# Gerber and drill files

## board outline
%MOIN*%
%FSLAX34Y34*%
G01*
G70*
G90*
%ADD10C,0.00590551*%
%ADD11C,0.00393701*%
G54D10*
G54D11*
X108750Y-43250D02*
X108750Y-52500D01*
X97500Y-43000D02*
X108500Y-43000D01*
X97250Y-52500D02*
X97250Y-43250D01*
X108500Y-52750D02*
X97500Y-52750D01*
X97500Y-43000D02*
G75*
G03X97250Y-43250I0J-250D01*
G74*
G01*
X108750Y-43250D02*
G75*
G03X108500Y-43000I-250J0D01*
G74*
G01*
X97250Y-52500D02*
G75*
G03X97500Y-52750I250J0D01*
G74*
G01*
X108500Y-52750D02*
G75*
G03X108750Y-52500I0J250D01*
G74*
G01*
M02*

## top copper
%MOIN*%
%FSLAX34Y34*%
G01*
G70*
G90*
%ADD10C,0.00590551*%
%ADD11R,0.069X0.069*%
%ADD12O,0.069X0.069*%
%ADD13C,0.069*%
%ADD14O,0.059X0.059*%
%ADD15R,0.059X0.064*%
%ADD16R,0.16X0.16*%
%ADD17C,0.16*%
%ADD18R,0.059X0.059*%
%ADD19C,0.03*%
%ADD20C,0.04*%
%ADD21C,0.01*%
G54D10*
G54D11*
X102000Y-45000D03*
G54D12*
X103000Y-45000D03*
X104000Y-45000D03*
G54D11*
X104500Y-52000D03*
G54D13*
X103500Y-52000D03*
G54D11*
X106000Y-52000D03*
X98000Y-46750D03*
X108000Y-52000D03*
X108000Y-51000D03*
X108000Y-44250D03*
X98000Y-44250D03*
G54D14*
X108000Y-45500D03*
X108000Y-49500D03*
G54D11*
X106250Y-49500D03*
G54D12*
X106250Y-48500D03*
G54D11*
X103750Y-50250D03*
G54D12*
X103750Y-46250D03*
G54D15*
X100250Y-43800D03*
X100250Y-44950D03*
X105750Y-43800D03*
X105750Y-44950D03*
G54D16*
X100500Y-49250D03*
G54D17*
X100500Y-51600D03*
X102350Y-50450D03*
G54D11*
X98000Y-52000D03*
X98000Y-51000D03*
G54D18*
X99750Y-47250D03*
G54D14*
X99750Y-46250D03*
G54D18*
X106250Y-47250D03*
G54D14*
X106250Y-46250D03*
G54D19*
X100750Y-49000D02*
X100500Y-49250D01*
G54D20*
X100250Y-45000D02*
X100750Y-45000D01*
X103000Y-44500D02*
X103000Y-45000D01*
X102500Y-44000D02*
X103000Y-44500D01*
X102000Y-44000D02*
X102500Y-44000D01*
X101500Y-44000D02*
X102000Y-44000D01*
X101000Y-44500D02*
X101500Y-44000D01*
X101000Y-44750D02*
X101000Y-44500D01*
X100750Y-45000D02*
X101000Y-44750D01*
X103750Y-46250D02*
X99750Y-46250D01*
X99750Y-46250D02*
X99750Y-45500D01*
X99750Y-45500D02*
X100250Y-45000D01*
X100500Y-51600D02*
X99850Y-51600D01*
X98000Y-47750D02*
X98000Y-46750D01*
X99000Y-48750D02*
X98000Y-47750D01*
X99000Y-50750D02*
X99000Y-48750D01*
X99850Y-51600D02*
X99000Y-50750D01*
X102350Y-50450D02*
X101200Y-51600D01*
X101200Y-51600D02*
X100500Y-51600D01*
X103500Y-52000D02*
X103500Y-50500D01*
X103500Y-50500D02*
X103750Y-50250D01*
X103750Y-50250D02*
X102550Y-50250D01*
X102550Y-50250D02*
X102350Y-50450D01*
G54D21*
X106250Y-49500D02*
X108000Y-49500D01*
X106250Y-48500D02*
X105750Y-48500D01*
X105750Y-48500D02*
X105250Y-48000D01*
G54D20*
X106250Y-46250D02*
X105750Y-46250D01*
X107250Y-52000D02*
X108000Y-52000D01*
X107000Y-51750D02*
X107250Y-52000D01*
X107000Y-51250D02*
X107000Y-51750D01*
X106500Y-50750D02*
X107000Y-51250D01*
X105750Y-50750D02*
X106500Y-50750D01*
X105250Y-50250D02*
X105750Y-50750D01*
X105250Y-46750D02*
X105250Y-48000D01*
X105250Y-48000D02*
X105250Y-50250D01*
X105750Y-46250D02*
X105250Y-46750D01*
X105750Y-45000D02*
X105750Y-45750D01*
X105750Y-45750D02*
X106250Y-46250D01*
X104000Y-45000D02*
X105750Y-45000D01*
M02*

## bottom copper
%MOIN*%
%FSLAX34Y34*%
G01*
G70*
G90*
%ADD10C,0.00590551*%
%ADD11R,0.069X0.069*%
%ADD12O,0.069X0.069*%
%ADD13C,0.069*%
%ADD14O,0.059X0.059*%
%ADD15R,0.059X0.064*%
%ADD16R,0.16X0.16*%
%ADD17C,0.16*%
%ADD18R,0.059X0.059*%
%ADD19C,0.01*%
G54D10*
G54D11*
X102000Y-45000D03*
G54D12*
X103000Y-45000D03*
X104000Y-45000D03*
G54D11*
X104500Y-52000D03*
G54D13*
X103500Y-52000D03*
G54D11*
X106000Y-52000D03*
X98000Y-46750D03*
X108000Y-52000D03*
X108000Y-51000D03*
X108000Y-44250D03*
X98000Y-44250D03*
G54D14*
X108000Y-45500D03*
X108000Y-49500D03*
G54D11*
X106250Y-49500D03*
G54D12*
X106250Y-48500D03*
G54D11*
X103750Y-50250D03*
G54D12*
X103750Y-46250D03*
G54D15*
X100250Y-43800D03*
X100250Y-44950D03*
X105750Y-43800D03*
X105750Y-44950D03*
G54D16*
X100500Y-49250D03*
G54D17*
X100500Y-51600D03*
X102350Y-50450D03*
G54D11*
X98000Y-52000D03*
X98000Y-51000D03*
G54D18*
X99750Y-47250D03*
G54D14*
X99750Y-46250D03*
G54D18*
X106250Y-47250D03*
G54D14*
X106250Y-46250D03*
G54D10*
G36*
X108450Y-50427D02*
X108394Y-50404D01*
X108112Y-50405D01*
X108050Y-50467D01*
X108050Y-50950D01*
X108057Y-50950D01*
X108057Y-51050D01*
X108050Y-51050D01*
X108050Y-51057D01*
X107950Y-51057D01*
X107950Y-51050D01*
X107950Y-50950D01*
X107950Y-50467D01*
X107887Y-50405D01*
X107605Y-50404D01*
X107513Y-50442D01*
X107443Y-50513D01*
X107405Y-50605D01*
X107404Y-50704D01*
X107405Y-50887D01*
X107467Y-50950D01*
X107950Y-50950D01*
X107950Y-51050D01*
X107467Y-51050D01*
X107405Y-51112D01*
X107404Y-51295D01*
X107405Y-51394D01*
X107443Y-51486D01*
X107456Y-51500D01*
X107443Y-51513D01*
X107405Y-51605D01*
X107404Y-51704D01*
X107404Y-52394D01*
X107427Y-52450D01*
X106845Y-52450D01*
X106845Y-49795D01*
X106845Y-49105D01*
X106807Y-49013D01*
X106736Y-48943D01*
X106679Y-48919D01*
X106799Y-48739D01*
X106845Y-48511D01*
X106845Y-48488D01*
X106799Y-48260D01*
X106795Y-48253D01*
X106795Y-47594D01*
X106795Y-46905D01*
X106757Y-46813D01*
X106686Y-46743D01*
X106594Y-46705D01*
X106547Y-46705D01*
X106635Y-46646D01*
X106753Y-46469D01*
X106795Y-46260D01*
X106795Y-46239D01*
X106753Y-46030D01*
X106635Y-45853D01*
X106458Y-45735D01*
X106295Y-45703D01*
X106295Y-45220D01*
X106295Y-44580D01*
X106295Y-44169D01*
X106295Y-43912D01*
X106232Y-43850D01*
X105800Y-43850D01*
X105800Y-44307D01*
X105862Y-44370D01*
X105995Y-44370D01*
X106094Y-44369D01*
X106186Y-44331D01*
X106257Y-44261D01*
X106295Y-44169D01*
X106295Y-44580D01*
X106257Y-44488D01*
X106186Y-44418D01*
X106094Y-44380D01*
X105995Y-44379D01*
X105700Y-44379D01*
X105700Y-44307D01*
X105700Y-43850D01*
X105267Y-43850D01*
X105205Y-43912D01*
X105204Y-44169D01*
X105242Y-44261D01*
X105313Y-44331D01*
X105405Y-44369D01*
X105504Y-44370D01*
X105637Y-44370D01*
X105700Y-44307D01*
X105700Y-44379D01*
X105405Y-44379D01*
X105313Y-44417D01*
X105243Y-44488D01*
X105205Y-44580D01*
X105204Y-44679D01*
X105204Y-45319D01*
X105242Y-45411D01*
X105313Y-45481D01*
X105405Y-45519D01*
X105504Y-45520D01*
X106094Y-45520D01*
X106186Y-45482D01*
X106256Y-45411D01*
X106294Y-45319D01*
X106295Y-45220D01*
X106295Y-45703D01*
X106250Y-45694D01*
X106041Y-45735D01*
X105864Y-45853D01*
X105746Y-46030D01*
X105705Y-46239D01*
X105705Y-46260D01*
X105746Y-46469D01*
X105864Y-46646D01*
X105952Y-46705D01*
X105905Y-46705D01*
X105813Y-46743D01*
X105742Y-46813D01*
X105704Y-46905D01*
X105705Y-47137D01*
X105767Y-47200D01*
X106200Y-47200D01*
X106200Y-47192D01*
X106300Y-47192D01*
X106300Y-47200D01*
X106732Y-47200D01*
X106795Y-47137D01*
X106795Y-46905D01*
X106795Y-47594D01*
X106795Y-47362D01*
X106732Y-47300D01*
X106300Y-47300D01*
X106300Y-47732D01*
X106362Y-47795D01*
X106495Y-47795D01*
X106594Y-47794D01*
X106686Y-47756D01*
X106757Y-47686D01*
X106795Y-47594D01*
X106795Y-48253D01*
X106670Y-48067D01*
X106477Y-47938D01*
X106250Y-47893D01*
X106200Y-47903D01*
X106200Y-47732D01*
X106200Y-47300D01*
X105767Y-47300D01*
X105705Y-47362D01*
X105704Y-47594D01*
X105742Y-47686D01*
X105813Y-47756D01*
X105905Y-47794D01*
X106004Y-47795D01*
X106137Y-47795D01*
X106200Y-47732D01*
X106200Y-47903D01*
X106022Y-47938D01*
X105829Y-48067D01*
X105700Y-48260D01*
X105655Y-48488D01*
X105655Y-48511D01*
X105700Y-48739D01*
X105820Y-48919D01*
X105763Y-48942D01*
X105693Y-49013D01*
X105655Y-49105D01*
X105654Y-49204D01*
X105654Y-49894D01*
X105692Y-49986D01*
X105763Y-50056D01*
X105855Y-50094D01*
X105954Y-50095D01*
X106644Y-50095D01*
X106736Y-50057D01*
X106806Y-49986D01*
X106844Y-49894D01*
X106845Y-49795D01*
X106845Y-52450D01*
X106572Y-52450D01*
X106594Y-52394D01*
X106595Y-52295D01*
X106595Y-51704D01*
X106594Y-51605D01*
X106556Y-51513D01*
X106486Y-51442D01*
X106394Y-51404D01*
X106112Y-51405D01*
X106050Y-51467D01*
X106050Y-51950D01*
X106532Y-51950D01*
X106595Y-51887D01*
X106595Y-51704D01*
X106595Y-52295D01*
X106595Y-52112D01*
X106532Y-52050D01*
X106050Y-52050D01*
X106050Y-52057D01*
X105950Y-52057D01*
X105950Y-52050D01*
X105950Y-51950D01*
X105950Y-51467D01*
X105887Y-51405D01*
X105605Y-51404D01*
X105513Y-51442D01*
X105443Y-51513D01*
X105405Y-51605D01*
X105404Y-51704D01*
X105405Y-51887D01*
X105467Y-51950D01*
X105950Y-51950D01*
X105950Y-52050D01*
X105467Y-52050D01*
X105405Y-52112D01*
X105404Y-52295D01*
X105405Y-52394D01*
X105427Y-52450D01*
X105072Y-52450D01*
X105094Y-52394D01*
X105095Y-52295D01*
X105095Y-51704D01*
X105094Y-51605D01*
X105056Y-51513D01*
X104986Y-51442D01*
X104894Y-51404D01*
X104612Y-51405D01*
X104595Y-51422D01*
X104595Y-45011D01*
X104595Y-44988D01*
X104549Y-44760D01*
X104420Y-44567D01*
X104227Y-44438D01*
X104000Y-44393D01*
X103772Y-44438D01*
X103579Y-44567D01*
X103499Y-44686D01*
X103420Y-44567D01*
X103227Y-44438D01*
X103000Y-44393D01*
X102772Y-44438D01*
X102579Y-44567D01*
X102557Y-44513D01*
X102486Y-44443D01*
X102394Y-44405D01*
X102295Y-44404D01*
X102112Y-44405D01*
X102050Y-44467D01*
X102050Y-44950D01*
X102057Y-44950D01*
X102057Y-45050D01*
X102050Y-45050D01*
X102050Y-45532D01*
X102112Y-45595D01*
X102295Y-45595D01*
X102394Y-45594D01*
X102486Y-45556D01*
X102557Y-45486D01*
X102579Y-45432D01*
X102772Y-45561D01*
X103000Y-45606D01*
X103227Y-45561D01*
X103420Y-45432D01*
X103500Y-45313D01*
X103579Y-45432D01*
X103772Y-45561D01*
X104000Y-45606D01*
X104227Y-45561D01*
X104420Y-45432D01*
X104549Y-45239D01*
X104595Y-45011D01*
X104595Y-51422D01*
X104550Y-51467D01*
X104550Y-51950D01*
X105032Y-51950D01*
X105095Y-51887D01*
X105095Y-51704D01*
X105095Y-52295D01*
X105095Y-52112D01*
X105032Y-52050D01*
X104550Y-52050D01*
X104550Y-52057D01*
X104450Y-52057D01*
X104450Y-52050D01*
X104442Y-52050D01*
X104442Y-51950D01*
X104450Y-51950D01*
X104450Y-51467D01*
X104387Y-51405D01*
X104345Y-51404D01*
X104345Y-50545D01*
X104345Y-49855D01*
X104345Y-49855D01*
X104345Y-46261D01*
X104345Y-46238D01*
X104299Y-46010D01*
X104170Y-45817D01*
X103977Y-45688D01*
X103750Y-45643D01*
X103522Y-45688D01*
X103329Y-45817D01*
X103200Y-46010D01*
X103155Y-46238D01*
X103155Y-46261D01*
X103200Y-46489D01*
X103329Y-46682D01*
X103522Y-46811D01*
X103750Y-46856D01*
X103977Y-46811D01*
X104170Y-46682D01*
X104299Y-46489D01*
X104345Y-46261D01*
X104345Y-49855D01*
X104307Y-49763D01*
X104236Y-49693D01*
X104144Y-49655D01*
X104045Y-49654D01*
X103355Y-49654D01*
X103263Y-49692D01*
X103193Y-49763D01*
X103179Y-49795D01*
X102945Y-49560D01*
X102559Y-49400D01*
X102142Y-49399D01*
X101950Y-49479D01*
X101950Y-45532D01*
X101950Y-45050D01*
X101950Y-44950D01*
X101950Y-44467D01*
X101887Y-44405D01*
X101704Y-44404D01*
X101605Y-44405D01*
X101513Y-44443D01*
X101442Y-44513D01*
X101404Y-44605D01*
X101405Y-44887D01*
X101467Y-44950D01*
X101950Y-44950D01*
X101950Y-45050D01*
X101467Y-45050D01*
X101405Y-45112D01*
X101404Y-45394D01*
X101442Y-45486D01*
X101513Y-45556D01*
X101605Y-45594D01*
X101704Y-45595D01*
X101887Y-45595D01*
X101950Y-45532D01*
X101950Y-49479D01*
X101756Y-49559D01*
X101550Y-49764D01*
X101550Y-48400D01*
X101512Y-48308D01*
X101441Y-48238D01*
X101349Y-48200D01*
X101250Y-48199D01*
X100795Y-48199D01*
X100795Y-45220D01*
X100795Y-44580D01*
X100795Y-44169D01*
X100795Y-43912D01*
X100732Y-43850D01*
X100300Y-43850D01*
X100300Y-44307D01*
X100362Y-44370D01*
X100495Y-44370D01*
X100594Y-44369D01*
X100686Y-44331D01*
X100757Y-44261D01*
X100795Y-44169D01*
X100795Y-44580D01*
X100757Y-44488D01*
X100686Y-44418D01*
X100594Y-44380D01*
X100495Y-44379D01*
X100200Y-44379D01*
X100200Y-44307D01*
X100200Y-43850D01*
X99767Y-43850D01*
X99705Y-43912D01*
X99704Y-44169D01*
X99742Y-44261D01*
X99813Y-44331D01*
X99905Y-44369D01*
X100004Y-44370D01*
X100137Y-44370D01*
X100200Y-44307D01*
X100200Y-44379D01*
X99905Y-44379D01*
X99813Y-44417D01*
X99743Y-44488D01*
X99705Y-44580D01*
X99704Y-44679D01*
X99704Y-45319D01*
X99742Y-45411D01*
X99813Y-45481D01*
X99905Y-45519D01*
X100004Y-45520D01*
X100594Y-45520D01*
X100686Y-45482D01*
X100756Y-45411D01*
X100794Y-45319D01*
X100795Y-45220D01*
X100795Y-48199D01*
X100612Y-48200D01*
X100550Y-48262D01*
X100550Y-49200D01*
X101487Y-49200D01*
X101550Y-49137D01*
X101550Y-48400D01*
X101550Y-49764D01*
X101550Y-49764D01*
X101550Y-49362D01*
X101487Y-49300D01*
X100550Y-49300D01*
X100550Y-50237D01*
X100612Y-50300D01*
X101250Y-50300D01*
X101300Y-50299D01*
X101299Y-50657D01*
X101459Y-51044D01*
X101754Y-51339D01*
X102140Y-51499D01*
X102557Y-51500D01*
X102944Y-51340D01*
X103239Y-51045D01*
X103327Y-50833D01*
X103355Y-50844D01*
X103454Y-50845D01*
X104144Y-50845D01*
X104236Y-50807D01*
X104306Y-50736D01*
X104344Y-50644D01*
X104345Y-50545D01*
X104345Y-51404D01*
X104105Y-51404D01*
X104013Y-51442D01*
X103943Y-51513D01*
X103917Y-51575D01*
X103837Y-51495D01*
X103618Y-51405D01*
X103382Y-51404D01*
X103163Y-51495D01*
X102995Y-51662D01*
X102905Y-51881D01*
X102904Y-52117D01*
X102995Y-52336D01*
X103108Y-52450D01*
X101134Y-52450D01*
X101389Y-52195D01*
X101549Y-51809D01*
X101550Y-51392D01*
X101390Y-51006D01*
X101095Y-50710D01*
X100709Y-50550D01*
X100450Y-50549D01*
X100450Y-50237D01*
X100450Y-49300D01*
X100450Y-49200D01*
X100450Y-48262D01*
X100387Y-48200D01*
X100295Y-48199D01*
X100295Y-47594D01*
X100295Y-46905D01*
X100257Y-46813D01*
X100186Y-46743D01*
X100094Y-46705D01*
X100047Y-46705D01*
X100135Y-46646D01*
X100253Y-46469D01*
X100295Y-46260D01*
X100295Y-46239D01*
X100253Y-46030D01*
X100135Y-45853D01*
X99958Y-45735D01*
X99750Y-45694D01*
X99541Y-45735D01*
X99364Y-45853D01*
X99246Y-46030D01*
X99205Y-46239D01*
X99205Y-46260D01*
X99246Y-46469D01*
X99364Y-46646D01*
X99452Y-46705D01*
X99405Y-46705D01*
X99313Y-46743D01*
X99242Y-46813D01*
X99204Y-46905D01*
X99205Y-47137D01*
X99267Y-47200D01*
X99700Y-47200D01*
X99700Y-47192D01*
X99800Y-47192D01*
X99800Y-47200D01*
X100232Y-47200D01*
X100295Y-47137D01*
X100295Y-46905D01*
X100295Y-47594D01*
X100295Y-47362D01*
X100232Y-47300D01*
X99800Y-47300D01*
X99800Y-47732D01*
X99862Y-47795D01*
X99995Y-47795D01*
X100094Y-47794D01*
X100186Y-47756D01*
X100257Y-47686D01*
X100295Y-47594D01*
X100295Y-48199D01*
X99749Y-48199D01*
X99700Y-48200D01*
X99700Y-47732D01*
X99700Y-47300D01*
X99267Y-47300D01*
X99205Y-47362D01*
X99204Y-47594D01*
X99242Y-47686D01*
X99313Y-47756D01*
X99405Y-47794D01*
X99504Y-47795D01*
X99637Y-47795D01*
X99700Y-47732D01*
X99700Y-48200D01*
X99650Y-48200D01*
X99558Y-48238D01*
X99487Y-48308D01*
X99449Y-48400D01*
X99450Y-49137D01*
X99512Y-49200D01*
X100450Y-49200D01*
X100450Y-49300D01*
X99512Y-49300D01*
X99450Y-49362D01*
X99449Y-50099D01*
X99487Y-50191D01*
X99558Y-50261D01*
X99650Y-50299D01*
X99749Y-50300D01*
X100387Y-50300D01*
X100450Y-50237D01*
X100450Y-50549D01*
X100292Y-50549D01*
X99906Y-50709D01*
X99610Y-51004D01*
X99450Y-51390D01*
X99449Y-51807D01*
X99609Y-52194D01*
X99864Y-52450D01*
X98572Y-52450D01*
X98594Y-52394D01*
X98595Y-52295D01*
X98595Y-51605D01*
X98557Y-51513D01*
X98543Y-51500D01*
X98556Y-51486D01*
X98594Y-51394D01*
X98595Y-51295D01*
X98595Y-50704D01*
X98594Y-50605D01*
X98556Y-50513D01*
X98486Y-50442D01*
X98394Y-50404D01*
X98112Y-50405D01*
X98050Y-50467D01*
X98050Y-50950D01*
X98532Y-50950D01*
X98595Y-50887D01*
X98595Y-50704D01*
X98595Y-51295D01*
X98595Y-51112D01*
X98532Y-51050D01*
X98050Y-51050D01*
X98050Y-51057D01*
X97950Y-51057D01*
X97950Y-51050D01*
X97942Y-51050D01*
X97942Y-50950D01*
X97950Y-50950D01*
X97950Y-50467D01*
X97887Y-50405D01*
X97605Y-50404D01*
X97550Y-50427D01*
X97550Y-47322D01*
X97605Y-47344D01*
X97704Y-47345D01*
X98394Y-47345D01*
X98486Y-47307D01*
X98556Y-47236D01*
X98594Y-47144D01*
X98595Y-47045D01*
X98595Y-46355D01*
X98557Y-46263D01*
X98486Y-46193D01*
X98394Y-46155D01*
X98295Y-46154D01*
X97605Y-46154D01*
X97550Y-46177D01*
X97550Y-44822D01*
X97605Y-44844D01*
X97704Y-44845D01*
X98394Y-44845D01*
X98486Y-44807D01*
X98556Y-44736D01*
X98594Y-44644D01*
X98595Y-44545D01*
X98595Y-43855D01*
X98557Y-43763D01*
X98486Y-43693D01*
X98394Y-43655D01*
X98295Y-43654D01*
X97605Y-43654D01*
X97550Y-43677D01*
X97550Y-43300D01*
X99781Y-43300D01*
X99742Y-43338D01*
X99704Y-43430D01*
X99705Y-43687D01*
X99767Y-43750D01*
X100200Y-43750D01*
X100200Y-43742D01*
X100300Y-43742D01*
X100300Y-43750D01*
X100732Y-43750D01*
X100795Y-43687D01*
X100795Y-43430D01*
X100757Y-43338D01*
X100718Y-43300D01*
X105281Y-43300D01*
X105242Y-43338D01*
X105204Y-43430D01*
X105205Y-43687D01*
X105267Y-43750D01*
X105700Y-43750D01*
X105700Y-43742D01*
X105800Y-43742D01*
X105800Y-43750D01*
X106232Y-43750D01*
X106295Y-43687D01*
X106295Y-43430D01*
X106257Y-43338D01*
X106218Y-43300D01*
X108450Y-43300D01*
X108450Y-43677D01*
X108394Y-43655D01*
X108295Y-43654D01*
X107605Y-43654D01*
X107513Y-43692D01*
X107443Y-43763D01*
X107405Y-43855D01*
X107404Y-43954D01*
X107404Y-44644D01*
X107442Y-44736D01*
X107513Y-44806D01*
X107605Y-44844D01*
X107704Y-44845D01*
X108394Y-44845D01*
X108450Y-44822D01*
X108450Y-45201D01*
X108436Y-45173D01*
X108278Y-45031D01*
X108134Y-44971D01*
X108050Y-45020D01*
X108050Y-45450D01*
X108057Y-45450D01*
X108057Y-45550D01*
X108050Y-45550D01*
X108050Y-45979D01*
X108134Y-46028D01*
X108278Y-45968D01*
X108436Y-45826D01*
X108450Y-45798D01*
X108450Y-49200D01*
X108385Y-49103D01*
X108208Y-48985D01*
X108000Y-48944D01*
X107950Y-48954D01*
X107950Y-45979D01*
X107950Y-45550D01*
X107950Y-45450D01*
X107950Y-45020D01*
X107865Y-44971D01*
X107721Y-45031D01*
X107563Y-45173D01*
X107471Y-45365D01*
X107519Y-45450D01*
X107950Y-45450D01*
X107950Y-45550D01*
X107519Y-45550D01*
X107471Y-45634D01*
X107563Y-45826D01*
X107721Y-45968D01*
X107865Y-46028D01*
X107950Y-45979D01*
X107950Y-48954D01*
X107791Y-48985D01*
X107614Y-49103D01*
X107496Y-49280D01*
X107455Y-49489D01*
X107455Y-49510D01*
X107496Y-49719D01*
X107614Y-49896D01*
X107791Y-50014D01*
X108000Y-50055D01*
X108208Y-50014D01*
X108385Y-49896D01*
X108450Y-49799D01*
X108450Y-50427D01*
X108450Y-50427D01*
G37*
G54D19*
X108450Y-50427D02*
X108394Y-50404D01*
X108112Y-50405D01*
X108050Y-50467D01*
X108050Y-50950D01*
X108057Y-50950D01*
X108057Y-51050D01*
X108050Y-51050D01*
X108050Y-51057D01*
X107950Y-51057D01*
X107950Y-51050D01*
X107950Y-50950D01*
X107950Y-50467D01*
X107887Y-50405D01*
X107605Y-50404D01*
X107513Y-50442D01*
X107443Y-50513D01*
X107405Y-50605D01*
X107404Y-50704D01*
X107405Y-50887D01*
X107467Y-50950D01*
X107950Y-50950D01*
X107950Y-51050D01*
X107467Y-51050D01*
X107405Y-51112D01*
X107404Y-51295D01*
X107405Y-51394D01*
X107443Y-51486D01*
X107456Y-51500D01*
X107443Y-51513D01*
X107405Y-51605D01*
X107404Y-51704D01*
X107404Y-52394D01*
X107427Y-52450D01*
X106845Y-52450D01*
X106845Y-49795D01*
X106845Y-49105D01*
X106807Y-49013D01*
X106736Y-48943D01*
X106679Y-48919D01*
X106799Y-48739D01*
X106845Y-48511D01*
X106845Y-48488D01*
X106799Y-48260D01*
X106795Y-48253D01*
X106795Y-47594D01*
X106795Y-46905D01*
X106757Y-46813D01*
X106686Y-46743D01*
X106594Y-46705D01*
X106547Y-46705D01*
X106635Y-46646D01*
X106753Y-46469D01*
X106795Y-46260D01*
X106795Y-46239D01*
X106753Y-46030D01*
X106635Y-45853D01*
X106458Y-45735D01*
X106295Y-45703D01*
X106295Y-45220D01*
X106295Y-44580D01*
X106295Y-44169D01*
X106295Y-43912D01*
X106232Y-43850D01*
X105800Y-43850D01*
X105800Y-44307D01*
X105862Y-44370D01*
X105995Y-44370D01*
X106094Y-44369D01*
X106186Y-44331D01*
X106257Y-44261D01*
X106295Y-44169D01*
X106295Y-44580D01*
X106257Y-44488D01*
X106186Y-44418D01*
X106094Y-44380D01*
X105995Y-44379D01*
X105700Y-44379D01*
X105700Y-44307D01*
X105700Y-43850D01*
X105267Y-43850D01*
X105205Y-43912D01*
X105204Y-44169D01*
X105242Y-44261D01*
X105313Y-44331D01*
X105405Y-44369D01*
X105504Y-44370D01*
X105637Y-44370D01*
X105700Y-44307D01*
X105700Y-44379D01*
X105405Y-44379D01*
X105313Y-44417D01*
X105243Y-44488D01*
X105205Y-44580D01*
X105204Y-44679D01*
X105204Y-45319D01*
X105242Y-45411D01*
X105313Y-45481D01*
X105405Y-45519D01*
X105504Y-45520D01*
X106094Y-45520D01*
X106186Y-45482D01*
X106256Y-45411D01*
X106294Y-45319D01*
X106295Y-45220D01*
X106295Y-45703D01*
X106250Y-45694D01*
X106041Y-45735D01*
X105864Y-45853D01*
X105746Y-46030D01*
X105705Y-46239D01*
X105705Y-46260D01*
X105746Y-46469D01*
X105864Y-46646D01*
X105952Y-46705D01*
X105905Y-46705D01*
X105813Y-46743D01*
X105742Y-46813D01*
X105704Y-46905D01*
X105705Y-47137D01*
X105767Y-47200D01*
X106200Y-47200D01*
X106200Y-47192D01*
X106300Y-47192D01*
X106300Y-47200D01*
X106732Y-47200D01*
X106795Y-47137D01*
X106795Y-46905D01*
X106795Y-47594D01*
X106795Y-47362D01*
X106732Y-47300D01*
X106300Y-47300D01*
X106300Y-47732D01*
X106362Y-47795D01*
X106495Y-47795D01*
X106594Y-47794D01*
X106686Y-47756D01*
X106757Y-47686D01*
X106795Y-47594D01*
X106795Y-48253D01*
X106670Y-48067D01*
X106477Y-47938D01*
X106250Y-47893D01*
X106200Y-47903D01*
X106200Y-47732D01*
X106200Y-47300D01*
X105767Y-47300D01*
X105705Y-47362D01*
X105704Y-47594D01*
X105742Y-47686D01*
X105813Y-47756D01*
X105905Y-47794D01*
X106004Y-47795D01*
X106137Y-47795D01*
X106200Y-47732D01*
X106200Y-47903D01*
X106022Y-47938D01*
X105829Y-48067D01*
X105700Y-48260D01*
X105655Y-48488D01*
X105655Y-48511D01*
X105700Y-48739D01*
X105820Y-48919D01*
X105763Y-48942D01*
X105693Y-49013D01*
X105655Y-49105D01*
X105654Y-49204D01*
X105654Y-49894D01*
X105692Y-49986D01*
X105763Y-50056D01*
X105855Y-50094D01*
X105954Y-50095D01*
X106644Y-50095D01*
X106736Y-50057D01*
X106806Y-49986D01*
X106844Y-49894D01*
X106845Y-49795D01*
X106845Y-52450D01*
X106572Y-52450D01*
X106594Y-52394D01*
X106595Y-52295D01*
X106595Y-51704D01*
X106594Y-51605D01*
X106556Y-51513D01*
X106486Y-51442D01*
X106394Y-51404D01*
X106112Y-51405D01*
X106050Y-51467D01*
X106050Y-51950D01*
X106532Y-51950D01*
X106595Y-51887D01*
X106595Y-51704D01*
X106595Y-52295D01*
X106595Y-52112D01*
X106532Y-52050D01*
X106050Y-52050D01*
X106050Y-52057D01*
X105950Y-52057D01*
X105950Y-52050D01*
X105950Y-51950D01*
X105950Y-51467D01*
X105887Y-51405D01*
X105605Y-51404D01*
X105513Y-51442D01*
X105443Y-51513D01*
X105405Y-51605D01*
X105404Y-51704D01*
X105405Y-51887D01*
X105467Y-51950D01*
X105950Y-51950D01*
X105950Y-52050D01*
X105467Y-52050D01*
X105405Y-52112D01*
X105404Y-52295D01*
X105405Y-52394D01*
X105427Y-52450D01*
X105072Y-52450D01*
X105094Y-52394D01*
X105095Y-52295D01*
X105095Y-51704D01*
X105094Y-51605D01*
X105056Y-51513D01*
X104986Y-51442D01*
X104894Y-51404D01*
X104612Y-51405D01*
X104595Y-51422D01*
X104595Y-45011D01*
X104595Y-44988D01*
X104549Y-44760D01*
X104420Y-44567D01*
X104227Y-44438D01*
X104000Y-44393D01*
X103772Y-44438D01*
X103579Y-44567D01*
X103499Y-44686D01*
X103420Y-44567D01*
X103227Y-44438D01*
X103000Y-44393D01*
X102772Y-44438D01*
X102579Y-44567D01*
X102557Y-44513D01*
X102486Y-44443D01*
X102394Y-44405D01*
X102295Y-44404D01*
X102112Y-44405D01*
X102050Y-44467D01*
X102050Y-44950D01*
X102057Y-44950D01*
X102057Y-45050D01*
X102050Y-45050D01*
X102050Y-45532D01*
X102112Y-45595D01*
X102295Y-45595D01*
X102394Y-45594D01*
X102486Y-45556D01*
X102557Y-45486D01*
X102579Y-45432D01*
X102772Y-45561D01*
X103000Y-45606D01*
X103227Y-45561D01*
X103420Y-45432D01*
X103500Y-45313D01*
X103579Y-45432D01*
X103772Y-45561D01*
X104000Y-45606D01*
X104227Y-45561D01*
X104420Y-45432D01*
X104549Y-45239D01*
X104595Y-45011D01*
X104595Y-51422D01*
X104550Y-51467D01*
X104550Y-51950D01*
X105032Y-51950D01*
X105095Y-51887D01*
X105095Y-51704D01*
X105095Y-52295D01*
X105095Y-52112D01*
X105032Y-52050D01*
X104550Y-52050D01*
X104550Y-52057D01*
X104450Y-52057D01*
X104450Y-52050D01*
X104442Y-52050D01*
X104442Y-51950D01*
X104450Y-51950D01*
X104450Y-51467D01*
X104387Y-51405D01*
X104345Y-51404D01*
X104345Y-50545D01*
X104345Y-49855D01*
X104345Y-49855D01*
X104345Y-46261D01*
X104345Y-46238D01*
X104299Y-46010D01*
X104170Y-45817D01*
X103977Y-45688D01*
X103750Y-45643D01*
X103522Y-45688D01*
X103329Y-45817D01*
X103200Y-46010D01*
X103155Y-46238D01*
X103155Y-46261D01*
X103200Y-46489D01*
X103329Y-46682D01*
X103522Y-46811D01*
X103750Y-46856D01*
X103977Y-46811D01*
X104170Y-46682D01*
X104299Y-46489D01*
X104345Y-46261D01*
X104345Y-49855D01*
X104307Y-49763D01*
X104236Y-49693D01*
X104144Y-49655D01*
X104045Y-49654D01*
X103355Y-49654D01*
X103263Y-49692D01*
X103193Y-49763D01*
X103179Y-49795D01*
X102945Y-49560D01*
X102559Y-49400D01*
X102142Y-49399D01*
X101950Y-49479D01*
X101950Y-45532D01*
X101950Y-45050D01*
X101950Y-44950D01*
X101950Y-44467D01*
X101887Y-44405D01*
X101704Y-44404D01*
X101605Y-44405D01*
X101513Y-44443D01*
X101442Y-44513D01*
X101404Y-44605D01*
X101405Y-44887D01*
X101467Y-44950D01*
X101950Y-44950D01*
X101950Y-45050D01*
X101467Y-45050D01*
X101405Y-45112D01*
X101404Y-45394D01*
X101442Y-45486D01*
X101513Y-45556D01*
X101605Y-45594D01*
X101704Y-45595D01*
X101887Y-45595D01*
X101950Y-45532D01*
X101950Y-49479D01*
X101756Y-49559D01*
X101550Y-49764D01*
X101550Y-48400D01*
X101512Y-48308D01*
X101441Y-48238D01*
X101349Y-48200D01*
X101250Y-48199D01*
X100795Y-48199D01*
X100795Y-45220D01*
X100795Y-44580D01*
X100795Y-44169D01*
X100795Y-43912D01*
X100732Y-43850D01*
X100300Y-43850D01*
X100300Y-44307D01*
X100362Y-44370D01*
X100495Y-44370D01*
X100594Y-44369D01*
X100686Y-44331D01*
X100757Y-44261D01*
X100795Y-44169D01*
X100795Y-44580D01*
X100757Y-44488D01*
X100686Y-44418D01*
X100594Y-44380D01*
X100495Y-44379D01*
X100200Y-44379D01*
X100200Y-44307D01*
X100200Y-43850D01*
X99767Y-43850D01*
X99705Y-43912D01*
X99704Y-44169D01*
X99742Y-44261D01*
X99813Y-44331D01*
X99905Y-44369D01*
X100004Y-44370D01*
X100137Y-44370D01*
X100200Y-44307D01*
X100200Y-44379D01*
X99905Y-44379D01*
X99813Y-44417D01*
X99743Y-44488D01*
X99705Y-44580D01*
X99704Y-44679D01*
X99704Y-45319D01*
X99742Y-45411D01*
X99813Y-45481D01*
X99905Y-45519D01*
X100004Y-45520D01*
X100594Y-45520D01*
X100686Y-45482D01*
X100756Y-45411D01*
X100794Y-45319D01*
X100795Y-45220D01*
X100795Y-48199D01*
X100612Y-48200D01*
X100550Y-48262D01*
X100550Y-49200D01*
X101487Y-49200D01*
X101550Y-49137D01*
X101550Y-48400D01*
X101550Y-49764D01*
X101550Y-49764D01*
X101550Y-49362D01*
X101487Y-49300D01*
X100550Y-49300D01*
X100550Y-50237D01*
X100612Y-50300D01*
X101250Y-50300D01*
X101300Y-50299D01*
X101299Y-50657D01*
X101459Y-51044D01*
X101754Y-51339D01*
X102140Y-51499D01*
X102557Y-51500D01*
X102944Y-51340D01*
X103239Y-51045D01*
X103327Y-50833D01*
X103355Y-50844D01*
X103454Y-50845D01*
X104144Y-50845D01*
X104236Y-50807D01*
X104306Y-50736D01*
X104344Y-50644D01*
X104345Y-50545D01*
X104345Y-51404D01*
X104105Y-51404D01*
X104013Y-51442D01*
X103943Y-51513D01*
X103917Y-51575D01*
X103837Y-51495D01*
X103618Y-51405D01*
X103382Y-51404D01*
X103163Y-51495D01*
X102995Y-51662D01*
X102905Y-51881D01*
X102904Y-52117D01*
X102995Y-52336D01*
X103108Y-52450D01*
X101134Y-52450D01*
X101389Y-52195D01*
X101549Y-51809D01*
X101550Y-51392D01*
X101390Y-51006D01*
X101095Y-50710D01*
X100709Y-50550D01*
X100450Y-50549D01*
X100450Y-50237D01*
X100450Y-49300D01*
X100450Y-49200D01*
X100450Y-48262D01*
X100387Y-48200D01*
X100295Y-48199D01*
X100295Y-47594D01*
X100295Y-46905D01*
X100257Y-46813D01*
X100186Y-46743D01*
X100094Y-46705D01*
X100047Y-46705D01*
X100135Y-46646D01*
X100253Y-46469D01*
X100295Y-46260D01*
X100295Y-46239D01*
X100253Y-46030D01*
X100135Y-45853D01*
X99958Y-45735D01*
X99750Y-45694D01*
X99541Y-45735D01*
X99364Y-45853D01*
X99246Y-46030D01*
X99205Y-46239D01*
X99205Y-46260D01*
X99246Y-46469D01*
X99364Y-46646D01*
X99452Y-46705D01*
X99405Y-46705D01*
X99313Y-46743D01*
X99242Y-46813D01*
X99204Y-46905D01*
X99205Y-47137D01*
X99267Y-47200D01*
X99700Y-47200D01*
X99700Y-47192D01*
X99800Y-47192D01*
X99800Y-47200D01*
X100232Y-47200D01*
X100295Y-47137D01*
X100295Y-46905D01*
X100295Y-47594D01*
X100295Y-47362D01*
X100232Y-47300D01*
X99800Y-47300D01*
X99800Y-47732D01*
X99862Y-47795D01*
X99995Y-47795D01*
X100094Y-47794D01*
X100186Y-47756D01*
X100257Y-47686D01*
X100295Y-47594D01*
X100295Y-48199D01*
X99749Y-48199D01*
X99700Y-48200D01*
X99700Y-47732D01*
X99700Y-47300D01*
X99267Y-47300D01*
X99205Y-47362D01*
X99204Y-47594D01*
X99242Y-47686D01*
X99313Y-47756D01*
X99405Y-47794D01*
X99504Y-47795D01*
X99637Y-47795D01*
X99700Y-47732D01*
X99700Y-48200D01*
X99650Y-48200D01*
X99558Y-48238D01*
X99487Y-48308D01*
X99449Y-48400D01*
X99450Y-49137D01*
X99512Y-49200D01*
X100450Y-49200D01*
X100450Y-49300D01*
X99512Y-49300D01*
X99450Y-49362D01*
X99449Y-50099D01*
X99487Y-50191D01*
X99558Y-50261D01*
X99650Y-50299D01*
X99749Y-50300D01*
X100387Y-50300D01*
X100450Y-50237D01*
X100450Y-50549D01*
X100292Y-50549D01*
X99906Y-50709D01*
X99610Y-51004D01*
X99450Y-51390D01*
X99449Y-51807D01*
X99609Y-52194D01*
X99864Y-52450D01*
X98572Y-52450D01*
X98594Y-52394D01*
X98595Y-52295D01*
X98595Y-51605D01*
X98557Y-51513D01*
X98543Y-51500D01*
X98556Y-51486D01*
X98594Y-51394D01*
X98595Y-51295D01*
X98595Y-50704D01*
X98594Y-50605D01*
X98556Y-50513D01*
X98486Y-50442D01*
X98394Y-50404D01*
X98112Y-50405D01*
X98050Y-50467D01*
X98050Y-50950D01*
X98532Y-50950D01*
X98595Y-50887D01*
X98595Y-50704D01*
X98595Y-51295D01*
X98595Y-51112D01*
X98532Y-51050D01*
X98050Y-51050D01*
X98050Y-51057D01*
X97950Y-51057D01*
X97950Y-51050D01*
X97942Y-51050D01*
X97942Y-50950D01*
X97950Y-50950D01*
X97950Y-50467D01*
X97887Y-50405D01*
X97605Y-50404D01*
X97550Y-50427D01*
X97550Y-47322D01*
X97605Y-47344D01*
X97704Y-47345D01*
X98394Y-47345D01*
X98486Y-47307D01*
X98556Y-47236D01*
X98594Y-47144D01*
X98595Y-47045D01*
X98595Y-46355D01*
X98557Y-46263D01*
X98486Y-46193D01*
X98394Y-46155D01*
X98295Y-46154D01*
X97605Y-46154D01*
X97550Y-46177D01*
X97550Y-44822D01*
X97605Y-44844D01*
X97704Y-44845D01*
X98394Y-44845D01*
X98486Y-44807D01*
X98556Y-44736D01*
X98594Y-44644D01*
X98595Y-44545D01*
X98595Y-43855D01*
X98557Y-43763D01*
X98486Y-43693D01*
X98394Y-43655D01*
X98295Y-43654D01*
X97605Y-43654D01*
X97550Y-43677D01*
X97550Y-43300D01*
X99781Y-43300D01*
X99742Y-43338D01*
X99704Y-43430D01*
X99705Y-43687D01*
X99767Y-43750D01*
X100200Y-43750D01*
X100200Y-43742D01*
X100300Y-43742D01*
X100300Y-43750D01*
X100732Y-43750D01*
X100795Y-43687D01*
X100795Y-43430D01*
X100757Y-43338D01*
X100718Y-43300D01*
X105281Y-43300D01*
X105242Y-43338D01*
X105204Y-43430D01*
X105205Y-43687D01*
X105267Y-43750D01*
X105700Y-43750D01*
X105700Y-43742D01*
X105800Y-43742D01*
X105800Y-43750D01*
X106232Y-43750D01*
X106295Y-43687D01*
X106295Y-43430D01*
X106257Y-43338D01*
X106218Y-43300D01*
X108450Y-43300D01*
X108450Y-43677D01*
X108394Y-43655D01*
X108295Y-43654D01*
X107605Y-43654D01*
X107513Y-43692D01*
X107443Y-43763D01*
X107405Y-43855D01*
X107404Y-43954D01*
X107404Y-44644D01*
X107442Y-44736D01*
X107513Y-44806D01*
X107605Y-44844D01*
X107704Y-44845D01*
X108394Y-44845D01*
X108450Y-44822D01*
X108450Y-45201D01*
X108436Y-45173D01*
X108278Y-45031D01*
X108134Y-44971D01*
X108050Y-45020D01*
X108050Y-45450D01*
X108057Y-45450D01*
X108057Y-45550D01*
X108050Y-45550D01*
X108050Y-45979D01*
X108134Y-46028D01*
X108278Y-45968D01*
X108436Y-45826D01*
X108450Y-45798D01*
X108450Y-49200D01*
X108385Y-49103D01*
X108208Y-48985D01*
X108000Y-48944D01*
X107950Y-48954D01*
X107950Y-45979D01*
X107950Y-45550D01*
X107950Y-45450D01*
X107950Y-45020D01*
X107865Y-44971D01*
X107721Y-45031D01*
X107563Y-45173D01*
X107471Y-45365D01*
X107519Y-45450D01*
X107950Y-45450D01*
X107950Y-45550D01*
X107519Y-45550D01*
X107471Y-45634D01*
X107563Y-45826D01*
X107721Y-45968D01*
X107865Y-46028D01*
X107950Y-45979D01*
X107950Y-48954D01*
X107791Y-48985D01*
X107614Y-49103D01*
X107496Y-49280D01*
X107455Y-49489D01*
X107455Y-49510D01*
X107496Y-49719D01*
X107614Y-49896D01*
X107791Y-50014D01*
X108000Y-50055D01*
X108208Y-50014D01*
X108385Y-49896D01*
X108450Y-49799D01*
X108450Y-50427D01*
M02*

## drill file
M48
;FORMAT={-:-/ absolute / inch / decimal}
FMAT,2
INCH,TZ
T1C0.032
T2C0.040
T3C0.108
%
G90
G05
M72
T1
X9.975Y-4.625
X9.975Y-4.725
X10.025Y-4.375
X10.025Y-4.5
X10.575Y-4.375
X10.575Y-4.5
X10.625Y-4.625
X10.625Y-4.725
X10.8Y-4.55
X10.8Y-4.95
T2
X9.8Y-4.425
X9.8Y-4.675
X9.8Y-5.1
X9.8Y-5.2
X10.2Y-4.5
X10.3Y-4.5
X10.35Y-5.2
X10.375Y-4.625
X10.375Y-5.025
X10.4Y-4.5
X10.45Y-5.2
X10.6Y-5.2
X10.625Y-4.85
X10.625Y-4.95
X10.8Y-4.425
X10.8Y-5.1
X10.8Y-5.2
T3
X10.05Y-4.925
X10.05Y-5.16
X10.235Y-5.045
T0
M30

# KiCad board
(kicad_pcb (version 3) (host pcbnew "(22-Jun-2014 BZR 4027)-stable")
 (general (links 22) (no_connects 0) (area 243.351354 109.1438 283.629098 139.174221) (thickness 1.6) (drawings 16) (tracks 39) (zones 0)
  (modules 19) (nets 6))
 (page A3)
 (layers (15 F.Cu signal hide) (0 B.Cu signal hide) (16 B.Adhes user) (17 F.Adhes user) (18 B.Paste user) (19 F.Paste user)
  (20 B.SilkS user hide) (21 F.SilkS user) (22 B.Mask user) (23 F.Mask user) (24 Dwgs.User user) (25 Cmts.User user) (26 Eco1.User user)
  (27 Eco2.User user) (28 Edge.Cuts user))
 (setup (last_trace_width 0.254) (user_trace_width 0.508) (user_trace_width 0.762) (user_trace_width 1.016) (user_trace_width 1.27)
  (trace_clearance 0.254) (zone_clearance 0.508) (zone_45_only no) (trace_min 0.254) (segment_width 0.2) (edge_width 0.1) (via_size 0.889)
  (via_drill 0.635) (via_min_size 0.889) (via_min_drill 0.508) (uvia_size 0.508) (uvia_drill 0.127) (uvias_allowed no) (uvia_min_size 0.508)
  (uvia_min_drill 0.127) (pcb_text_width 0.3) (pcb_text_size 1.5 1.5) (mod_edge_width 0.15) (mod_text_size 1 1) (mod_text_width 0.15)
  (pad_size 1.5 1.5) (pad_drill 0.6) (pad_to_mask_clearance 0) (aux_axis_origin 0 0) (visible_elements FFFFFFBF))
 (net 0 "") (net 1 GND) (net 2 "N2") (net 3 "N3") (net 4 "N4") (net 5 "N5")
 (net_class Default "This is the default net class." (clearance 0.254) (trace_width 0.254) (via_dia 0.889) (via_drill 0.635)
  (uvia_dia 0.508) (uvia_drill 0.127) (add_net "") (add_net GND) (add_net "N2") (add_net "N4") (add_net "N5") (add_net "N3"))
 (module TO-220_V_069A (layer F.Cu) (at 259.08 114.3)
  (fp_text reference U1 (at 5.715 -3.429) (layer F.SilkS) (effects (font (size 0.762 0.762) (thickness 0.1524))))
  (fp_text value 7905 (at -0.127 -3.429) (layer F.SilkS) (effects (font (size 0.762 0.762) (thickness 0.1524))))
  (pad 1 thru_hole rect (at 0 0 90) (size 1.7526 1.7526) (drill 1.016) (layers *.Cu *.Mask F.SilkS) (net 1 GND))
  (pad 2 thru_hole oval (at 2.54 0 90) (size 1.7526 1.7526) (drill 1.016) (layers *.Cu *.Mask F.SilkS) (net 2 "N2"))
  (pad 3 thru_hole oval (at 5.08 0 90) (size 1.7526 1.7526) (drill 1.016) (layers *.Cu *.Mask F.SilkS) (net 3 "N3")))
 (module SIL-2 (layer F.Cu) (at 265.43 132.08 180)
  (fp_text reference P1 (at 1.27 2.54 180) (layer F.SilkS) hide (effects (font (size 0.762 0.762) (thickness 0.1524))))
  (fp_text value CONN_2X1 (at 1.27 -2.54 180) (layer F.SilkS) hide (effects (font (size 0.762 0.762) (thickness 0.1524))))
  (pad 1 thru_hole rect (at 0 0 180) (size 1.7526 1.7526) (drill 1.016) (layers *.Cu *.Mask F.SilkS) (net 1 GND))
  (pad 2 thru_hole circle (at 2.54 0 180) (size 1.7526 1.7526) (drill 1.016) (layers *.Cu *.Mask F.SilkS) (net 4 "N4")))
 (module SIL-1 (layer F.Cu) (at 269.24 132.08 180)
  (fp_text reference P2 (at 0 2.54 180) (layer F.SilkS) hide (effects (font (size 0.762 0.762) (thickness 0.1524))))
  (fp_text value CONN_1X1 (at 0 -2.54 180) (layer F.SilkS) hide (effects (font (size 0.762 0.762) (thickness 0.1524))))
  (pad 1 thru_hole rect (at 0 0 180) (size 1.7526 1.7526) (drill 1.016) (layers *.Cu *.Mask F.SilkS) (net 1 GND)))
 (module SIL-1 (layer F.Cu) (at 248.92 118.745 180)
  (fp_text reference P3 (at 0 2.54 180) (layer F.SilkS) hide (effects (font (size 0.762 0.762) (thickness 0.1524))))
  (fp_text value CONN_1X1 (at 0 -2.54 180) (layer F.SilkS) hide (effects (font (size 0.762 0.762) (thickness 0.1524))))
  (pad 1 thru_hole rect (at 0 0 180) (size 1.7526 1.7526) (drill 1.016) (layers *.Cu *.Mask F.SilkS) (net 4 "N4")))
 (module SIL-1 (layer F.Cu) (at 274.32 132.08 180)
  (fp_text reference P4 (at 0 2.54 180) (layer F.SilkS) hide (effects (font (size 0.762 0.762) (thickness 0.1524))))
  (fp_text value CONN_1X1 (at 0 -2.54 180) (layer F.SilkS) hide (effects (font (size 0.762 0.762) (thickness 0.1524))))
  (pad 1 thru_hole rect (at 0 0 180) (size 1.7526 1.7526) (drill 1.016) (layers *.Cu *.Mask F.SilkS) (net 3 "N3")))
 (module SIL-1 (layer F.Cu) (at 274.32 129.54 180)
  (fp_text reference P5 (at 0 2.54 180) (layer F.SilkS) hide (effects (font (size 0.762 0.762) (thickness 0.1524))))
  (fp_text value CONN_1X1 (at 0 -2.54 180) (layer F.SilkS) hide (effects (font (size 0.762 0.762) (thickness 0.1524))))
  (pad 1 thru_hole rect (at 0 0 180) (size 1.7526 1.7526) (drill 1.016) (layers *.Cu *.Mask F.SilkS) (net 1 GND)))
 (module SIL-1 (layer F.Cu) (at 274.32 112.395 180)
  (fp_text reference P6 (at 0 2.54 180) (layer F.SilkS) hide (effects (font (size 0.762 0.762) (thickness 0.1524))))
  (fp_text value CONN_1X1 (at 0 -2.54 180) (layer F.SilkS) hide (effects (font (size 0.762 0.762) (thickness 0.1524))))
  (pad 1 thru_hole rect (at 0 0 180) (size 1.7526 1.7526) (drill 1.016) (layers *.Cu *.Mask F.SilkS)))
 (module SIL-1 (layer F.Cu) (at 248.92 112.395 180)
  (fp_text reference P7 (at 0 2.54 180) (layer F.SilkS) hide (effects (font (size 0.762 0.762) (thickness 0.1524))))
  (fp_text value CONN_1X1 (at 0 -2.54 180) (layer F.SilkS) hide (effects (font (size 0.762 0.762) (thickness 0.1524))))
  (pad 1 thru_hole rect (at 0 0 180) (size 1.7526 1.7526) (drill 1.016) (layers *.Cu *.Mask F.SilkS)))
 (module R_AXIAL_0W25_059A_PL (layer F.Cu) (at 274.32 115.57 270) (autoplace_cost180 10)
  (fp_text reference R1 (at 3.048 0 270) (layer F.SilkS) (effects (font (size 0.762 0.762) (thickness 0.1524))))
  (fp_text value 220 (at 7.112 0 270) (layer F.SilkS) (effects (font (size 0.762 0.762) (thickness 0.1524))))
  (pad 1 thru_hole oval (at 0 0 270) (size 1.4986 1.4986) (drill 0.8128) (layers *.Cu *.Mask F.SilkS) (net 1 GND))
  (pad 2 thru_hole oval (at 10.16 0 270) (size 1.4986 1.4986) (drill 0.8128) (layers *.Cu *.Mask F.SilkS) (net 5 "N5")))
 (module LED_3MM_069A (layer F.Cu) (at 269.875 125.73 90)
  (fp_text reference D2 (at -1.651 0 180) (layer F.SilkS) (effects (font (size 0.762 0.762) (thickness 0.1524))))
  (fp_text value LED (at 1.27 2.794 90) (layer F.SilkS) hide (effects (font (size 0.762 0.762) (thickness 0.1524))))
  (pad 1 thru_hole rect (at 0 0 90) (size 1.7526 1.7526) (drill 1.016) (layers *.Cu *.Mask F.SilkS) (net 5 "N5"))
  (pad 2 thru_hole oval (at 2.54 0 90) (size 1.7526 1.7526) (drill 1.016) (layers *.Cu *.Mask F.SilkS) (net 3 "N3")))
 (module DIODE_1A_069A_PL (layer F.Cu) (at 263.525 122.555 270)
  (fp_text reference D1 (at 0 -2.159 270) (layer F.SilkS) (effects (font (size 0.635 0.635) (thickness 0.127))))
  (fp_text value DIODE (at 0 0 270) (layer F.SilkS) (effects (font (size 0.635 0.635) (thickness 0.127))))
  (pad 2 thru_hole rect (at 5.08 0 270) (size 1.7526 1.7526) (drill 1.016) (layers *.Cu *.Mask F.SilkS) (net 4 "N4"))
  (pad 1 thru_hole oval (at -5.08 0 270) (size 1.7526 1.7526) (drill 1.016) (layers *.Cu *.Mask F.SilkS) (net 2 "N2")))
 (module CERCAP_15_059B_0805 (layer F.Cu) (at 254.635 111.125 270)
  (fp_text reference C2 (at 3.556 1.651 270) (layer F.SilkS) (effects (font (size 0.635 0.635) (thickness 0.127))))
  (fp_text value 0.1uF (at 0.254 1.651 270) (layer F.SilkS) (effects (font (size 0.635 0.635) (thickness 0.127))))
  (pad 1 thru_hole rect (at 0 0 270) (size 1.6256 1.4986) (drill 0.8128 (offset 0.127 0)) (layers *.Cu *.Mask F.SilkS) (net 1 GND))
  (pad 2 thru_hole rect (at 3.175 0 270) (size 1.6256 1.4986) (drill 0.8128 (offset -0.127 0)) (layers *.Cu *.Mask F.SilkS) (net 2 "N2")))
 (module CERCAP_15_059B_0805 (layer F.Cu) (at 268.605 111.125 270)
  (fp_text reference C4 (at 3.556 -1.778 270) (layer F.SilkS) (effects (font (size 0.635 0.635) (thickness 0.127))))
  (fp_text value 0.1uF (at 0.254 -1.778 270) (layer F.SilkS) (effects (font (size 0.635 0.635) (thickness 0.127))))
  (pad 1 thru_hole rect (at 0 0 270) (size 1.6256 1.4986) (drill 0.8128 (offset 0.127 0)) (layers *.Cu *.Mask F.SilkS) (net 1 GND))
  (pad 2 thru_hole rect (at 3.175 0 270) (size 1.6256 1.4986) (drill 0.8128 (offset -0.127 0)) (layers *.Cu *.Mask F.SilkS) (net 3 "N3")))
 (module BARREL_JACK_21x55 (layer F.Cu) (at 255.27 125.095 90)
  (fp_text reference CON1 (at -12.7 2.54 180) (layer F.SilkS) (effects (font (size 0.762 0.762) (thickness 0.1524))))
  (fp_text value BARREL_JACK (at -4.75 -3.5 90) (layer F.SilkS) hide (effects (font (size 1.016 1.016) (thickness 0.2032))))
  (pad 1 thru_hole rect (at 0 0 90) (size 4.064 4.064) (drill 2.7432) (layers *.Cu *.Mask F.SilkS) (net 1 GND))
  (pad 2 thru_hole circle (at -5.969 0 90) (size 4.064 4.064) (drill 2.7432) (layers *.Cu *.Mask F.SilkS) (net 4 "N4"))
  (pad 3 thru_hole circle (at -3.048 4.699 90) (size 4.064 4.064) (drill 2.7432) (layers *.Cu *.Mask F.SilkS) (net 4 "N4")))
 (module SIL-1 (layer F.Cu) (at 248.92 132.08 180)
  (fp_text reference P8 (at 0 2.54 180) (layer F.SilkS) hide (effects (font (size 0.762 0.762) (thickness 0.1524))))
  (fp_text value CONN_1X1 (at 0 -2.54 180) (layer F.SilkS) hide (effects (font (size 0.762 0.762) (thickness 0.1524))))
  (pad 1 thru_hole rect (at 0 0 180) (size 1.7526 1.7526) (drill 1.016) (layers *.Cu *.Mask F.SilkS)))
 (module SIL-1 (layer F.Cu) (at 248.92 129.54 180)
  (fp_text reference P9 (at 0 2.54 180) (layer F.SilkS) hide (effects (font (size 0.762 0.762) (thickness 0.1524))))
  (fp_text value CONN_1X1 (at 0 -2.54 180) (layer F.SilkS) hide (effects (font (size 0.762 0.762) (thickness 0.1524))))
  (pad 1 thru_hole rect (at 0 0 180) (size 1.7526 1.7526) (drill 1.016) (layers *.Cu *.Mask F.SilkS) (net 1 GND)))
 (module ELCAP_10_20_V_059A (layer F.Cu) (at 253.365 120.015 90)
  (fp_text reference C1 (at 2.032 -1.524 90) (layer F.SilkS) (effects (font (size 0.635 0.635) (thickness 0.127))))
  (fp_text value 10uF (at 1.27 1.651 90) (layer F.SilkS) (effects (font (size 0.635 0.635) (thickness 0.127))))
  (pad 1 thru_hole rect (at 0 0 90) (size 1.4986 1.4986) (drill 0.8128) (layers *.Cu *.Mask F.SilkS) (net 1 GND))
  (pad 2 thru_hole oval (at 2.54 0 90) (size 1.4986 1.4986) (drill 0.8128) (layers *.Cu *.Mask F.SilkS) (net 2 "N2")))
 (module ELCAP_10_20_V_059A (layer F.Cu) (at 269.875 120.015 90)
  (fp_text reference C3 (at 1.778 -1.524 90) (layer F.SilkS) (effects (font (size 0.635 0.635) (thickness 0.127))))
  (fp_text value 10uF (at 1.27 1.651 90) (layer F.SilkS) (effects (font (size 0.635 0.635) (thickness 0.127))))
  (pad 1 thru_hole rect (at 0 0 90) (size 1.4986 1.4986) (drill 0.8128) (layers *.Cu *.Mask F.SilkS) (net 1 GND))
  (pad 2 thru_hole oval (at 2.54 0 90) (size 1.4986 1.4986) (drill 0.8128) (layers *.Cu *.Mask F.SilkS) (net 3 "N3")))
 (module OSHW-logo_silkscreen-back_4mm (layer F.Cu) (at 261.62 121.285 90)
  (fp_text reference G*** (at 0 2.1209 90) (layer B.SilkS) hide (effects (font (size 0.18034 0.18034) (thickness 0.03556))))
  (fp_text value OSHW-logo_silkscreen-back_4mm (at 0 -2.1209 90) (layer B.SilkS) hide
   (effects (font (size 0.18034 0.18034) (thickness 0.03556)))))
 (gr_line (start 276.225 109.855) (end 276.225 133.35) (angle 90) (layer Edge.Cuts) (width 0.1))
 (gr_line (start 247.65 109.22) (end 275.59 109.22) (angle 90) (layer Edge.Cuts) (width 0.1))
 (gr_line (start 247.015 133.35) (end 247.015 109.855) (angle 90) (layer Edge.Cuts) (width 0.1))
 (gr_line (start 275.59 133.985) (end 247.65 133.985) (angle 90) (layer Edge.Cuts) (width 0.1))
 (gr_arc (start 247.65 109.855) (end 247.015 109.855) (angle 90) (layer Edge.Cuts) (width 0.1))
 (gr_arc (start 275.59 109.855) (end 275.59 109.22) (angle 90) (layer Edge.Cuts) (width 0.1))
 (gr_arc (start 247.65 133.35) (end 247.65 133.985) (angle 90) (layer Edge.Cuts) (width 0.1))
 (gr_arc (start 275.59 133.35) (end 276.225 133.35) (angle 90) (layer Edge.Cuts) (width 0.1))
 (segment (start 255.905 124.46) (end 255.27 125.095) (width 0.762) (layer F.Cu) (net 1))
 (segment (start 254.635 114.3) (end 255.905 114.3) (width 1.016) (layer F.Cu) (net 2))
 (segment (start 261.62 113.03) (end 261.62 114.3) (width 1.016) (layer F.Cu) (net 2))
 (segment (start 260.35 111.76) (end 261.62 113.03) (width 1.016) (layer F.Cu) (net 2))
 (segment (start 259.08 111.76) (end 260.35 111.76) (width 1.016) (layer F.Cu) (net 2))
 (segment (start 257.81 111.76) (end 259.08 111.76) (width 1.016) (layer F.Cu) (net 2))
 (segment (start 256.54 113.03) (end 257.81 111.76) (width 1.016) (layer F.Cu) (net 2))
 (segment (start 256.54 113.665) (end 256.54 113.03) (width 1.016) (layer F.Cu) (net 2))
 (segment (start 255.905 114.3) (end 256.54 113.665) (width 1.016) (layer F.Cu) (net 2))
 (segment (start 263.525 117.475) (end 253.365 117.475) (width 1.016) (layer F.Cu) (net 2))
 (segment (start 253.365 117.475) (end 253.365 115.57) (width 1.016) (layer F.Cu) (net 2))
 (segment (start 253.365 115.57) (end 254.635 114.3) (width 1.016) (layer F.Cu) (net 2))
 (segment (start 255.27 131.064) (end 253.619 131.064) (width 1.016) (layer F.Cu) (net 4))
 (segment (start 248.92 121.285) (end 248.92 118.745) (width 1.016) (layer F.Cu) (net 4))
 (segment (start 251.46 123.825) (end 248.92 121.285) (width 1.016) (layer F.Cu) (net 4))
 (segment (start 251.46 128.905) (end 251.46 123.825) (width 1.016) (layer F.Cu) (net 4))
 (segment (start 253.619 131.064) (end 251.46 128.905) (width 1.016) (layer F.Cu) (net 4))
 (segment (start 259.969 128.143) (end 257.048 131.064) (width 1.016) (layer F.Cu) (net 4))
 (segment (start 257.048 131.064) (end 255.27 131.064) (width 1.016) (layer F.Cu) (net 4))
 (segment (start 262.89 132.08) (end 262.89 128.27) (width 1.016) (layer F.Cu) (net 4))
 (segment (start 262.89 128.27) (end 263.525 127.635) (width 1.016) (layer F.Cu) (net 4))
 (segment (start 263.525 127.635) (end 260.477 127.635) (width 1.016) (layer F.Cu) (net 4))
 (segment (start 260.477 127.635) (end 259.969 128.143) (width 1.016) (layer F.Cu) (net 4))
 (segment (start 269.875 125.73) (end 274.32 125.73) (width 0.254) (layer F.Cu) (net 5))
 (segment (start 269.875 123.19) (end 268.605 123.19) (width 0.254) (layer F.Cu) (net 3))
 (segment (start 268.605 123.19) (end 267.335 121.92) (width 0.254) (layer F.Cu) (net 3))
 (segment (start 269.875 117.475) (end 268.605 117.475) (width 1.016) (layer F.Cu) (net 3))
 (segment (start 272.415 132.08) (end 274.32 132.08) (width 1.016) (layer F.Cu) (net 3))
 (segment (start 271.78 131.445) (end 272.415 132.08) (width 1.016) (layer F.Cu) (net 3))
 (segment (start 271.78 130.175) (end 271.78 131.445) (width 1.016) (layer F.Cu) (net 3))
 (segment (start 270.51 128.905) (end 271.78 130.175) (width 1.016) (layer F.Cu) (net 3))
 (segment (start 268.605 128.905) (end 270.51 128.905) (width 1.016) (layer F.Cu) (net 3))
 (segment (start 267.335 127.635) (end 268.605 128.905) (width 1.016) (layer F.Cu) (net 3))
 (segment (start 267.335 118.745) (end 267.335 121.92) (width 1.016) (layer F.Cu) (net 3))
 (segment (start 267.335 121.92) (end 267.335 127.635) (width 1.016) (layer F.Cu) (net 3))
 (segment (start 268.605 117.475) (end 267.335 118.745) (width 1.016) (layer F.Cu) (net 3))
 (segment (start 268.605 114.3) (end 268.605 116.205) (width 1.016) (layer F.Cu) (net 3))
 (segment (start 268.605 116.205) (end 269.875 117.475) (width 1.016) (layer F.Cu) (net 3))
 (segment (start 264.16 114.3) (end 268.605 114.3) (width 1.016) (layer F.Cu) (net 3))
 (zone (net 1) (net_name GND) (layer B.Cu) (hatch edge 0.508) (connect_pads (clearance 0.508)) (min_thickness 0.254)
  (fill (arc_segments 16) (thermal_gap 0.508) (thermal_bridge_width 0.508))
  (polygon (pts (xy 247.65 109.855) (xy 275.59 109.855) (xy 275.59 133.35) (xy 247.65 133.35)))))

